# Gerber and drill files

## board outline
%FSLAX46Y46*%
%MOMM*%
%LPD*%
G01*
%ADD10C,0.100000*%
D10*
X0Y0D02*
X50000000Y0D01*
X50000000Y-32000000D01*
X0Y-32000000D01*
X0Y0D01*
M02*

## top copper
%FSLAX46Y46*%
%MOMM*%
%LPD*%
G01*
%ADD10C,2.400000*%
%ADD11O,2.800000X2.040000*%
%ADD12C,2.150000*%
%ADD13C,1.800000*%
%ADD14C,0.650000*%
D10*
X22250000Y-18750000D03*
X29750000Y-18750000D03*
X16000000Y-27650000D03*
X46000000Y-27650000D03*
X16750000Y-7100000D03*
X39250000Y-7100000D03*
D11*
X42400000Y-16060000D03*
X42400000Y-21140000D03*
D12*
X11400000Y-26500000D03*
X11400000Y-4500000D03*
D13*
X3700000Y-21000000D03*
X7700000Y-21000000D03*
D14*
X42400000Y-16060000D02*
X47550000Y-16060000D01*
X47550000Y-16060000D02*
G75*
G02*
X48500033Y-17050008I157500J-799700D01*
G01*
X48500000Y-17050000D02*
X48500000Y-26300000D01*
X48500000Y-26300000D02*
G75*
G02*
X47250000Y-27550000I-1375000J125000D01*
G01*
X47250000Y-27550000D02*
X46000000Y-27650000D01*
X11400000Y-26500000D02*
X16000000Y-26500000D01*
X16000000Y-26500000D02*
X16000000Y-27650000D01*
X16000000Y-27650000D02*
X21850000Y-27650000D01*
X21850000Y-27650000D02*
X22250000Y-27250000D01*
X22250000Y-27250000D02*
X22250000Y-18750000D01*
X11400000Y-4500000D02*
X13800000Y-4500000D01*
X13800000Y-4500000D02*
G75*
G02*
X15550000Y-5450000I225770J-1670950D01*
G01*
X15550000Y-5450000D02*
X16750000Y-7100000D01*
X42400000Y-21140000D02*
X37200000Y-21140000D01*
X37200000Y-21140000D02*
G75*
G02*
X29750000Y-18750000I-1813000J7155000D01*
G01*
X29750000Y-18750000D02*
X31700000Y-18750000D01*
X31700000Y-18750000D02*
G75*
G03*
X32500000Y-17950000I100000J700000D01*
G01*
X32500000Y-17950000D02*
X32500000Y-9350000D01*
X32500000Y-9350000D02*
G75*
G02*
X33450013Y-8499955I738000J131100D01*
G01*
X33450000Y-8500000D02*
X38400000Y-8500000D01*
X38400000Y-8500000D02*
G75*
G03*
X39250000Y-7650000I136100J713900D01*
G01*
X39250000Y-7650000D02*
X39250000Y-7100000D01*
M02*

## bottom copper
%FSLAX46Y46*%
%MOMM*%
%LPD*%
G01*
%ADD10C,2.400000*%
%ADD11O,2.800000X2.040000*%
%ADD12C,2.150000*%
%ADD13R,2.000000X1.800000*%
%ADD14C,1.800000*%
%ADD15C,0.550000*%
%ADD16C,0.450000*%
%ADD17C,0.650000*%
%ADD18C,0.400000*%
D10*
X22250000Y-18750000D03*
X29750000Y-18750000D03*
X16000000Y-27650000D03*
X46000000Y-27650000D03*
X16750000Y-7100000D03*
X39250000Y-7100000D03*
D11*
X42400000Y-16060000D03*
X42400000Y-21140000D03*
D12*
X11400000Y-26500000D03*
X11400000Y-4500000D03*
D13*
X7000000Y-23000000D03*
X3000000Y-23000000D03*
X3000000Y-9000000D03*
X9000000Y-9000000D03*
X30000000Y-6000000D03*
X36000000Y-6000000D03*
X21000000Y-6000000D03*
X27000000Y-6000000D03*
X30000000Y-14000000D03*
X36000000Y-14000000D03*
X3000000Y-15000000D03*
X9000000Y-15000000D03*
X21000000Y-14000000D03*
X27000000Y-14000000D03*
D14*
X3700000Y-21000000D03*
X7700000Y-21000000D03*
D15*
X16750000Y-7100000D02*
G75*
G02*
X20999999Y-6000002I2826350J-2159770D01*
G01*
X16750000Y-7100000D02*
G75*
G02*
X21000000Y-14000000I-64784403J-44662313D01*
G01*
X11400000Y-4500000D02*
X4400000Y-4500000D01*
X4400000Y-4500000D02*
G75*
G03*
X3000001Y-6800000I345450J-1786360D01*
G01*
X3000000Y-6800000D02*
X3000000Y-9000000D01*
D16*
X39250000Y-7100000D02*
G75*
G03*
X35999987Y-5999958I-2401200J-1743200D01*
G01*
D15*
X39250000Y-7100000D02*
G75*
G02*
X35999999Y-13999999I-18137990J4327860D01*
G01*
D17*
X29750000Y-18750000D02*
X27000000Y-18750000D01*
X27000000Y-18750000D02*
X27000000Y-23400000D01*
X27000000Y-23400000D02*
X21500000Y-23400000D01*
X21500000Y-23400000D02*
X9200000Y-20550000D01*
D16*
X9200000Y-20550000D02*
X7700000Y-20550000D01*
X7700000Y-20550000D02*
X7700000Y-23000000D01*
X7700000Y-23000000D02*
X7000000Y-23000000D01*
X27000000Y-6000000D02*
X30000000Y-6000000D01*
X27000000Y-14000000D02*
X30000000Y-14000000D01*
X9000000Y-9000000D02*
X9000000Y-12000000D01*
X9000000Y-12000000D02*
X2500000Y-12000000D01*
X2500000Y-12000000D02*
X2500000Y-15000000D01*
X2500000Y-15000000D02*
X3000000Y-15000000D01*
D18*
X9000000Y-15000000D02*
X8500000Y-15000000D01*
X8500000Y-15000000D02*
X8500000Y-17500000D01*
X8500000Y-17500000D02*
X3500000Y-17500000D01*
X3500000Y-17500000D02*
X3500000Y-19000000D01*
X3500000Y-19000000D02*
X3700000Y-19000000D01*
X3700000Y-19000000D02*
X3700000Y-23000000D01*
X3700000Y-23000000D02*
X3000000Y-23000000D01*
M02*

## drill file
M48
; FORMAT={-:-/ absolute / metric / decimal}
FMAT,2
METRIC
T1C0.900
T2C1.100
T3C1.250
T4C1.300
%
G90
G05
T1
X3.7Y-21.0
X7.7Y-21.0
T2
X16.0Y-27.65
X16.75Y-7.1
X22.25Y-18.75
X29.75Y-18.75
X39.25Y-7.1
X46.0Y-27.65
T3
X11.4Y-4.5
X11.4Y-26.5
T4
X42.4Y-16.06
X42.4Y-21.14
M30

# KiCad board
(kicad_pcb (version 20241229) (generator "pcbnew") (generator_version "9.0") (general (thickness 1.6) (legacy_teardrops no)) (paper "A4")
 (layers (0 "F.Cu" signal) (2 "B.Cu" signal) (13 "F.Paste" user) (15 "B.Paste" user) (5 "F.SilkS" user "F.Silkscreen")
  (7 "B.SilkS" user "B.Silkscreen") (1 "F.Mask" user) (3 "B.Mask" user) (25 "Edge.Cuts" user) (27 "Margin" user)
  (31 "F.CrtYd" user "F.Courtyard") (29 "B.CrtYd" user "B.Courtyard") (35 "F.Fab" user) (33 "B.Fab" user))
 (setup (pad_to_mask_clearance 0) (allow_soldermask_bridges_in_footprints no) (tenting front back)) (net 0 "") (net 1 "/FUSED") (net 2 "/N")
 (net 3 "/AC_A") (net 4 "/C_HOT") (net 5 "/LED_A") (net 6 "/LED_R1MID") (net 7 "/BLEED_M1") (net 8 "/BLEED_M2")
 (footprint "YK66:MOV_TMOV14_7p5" (layer "F.Cu") (at 26 18.75)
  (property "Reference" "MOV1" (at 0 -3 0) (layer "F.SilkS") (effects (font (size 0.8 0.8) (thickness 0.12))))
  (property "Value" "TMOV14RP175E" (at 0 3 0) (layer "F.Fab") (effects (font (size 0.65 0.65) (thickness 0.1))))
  (pad "1" thru_hole circle (at -3.75 0) (size 2.4 2.4) (drill 1.1) (layers "*.Cu" "*.Mask") (remove_unused_layers no) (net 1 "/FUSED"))
  (pad "2" thru_hole circle (at 3.75 0) (size 2.4 2.4) (drill 1.1) (layers "*.Cu" "*.Mask") (remove_unused_layers no) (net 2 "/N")))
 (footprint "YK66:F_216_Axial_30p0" (layer "F.Cu") (at 31 27.65)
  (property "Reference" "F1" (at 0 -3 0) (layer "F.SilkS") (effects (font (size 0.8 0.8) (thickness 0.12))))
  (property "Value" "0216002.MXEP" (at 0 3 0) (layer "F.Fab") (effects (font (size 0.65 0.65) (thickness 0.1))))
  (pad "1" thru_hole circle (at -15 0) (size 2.4 2.4) (drill 1.1) (layers "*.Cu" "*.Mask") (remove_unused_layers no) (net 1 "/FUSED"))
  (pad "2" thru_hole circle (at 15 0) (size 2.4 2.4) (drill 1.1) (layers "*.Cu" "*.Mask") (remove_unused_layers no) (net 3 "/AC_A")))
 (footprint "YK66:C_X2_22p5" (layer "F.Cu") (at 28 7.1)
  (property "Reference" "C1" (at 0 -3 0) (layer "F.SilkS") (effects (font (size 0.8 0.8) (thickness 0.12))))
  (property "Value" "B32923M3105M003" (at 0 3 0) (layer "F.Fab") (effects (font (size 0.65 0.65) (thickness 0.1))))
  (pad "1" thru_hole circle (at -11.25 0) (size 2.4 2.4) (drill 1.1) (layers "*.Cu" "*.Mask") (remove_unused_layers no) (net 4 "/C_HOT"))
  (pad "2" thru_hole circle (at 11.25 0) (size 2.4 2.4) (drill 1.1) (layers "*.Cu" "*.Mask") (remove_unused_layers no) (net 2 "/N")))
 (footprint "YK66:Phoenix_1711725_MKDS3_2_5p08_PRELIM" (layer "F.Cu") (at 42.4 18.6)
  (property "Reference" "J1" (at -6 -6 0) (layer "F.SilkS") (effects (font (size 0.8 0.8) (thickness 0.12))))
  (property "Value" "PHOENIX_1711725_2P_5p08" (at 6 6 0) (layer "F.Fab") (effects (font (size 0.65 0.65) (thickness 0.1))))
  (pad "1" thru_hole oval (at 0 -2.54) (size 2.8 2.04) (drill 1.3) (layers "*.Cu" "*.Mask") (remove_unused_layers no) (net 3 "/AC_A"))
  (pad "2" thru_hole oval (at 0 2.54) (size 2.8 2.04) (drill 1.3) (layers "*.Cu" "*.Mask") (remove_unused_layers no) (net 2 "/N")))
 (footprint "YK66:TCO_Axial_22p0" (layer "F.Cu") (at 11.4 15.5)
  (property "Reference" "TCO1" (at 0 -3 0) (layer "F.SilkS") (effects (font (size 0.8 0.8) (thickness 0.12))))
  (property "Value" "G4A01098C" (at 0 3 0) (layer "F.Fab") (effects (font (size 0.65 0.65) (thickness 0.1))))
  (pad "1" thru_hole circle (at 0 11) (size 2.15 2.15) (drill 1.25) (layers "*.Cu" "*.Mask") (remove_unused_layers no) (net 1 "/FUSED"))
  (pad "2" thru_hole circle (at 0 -11) (size 2.15 2.15) (drill 1.25) (layers "*.Cu" "*.Mask") (remove_unused_layers no) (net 4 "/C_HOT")))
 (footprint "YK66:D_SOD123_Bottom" (layer "B.Cu") (at 5 23)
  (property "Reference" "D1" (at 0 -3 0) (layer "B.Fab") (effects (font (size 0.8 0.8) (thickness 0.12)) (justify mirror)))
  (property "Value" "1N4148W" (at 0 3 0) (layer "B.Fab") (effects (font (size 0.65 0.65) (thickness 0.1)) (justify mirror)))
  (pad "1" smd rect (at 2 0) (size 2 1.8) (layers "B.Cu" "B.Mask" "B.Paste") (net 2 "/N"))
  (pad "2" smd rect (at -2 0) (size 2 1.8) (layers "B.Cu" "B.Mask" "B.Paste") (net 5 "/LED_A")))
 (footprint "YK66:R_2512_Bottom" (layer "B.Cu") (at 6 9)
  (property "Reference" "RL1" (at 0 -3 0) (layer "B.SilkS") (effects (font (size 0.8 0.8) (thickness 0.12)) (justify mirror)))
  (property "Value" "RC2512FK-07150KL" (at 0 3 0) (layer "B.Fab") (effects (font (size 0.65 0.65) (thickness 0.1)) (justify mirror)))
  (pad "1" smd rect (at -3 0) (size 2 1.8) (layers "B.Cu" "B.Mask" "B.Paste") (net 4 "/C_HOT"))
  (pad "2" smd rect (at 3 0) (size 2 1.8) (layers "B.Cu" "B.Mask" "B.Paste") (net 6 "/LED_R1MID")))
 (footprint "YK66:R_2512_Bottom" (layer "B.Cu") (at 33 6)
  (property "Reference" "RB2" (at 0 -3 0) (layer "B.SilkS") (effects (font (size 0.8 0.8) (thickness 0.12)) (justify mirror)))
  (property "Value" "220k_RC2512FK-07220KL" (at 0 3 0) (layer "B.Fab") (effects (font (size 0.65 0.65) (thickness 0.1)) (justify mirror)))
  (pad "1" smd rect (at -3 0) (size 2 1.8) (layers "B.Cu" "B.Mask" "B.Paste") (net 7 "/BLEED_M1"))
  (pad "2" smd rect (at 3 0) (size 2 1.8) (layers "B.Cu" "B.Mask" "B.Paste") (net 2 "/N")))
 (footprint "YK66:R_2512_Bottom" (layer "B.Cu") (at 24 6)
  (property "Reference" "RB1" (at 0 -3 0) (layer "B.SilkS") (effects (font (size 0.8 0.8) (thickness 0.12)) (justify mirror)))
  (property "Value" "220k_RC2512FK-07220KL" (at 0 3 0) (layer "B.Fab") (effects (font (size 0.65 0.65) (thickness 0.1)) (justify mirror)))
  (pad "1" smd rect (at -3 0) (size 2 1.8) (layers "B.Cu" "B.Mask" "B.Paste") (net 4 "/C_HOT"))
  (pad "2" smd rect (at 3 0) (size 2 1.8) (layers "B.Cu" "B.Mask" "B.Paste") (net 7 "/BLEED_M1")))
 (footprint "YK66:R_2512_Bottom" (layer "B.Cu") (at 33 14)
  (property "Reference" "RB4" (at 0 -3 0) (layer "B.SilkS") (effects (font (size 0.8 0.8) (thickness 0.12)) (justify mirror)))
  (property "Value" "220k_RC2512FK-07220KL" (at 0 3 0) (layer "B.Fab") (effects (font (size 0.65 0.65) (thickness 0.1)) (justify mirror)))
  (pad "1" smd rect (at -3 0) (size 2 1.8) (layers "B.Cu" "B.Mask" "B.Paste") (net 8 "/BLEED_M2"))
  (pad "2" smd rect (at 3 0) (size 2 1.8) (layers "B.Cu" "B.Mask" "B.Paste") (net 2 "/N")))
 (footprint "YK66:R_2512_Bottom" (layer "B.Cu") (at 6 15)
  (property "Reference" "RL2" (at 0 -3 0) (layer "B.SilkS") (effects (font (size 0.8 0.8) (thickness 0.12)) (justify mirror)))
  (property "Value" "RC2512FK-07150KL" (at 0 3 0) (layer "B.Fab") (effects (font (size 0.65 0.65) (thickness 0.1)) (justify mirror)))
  (pad "1" smd rect (at -3 0) (size 2 1.8) (layers "B.Cu" "B.Mask" "B.Paste") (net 6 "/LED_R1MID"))
  (pad "2" smd rect (at 3 0) (size 2 1.8) (layers "B.Cu" "B.Mask" "B.Paste") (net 5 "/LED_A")))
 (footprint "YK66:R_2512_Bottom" (layer "B.Cu") (at 24 14)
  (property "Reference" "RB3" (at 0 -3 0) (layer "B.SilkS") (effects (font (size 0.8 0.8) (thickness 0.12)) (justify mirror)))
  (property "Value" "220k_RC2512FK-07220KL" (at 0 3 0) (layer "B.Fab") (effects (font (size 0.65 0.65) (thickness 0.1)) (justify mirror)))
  (pad "1" smd rect (at -3 0) (size 2 1.8) (layers "B.Cu" "B.Mask" "B.Paste") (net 4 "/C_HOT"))
  (pad "2" smd rect (at 3 0) (size 2 1.8) (layers "B.Cu" "B.Mask" "B.Paste") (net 8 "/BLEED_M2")))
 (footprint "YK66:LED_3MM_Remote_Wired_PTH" (layer "F.Cu") (at 5.7 21)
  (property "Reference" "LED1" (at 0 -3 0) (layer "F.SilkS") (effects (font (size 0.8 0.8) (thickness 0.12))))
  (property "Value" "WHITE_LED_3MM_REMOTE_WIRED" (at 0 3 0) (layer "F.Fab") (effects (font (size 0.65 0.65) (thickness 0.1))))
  (pad "1" thru_hole circle (at -2 0) (size 1.8 1.8) (drill 0.9) (layers "*.Cu" "*.Mask") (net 5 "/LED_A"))
  (pad "2" thru_hole circle (at 2 0) (size 1.8 1.8) (drill 0.9) (layers "*.Cu" "*.Mask") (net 2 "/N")))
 (gr_rect (start 0 0) (end 50 32) (stroke (width 0.1) (type default)) (fill no) (layer "Edge.Cuts"))
 (segment (start 42.4000 16.0600) (end 47.5500 16.0600) (width 0.650) (layer "F.Cu") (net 3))
 (arc (start 47.5500 16.0600) (mid 48.3000 16.3000) (end 48.5000 17.0500) (width 0.650) (layer "F.Cu") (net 3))
 (segment (start 48.5000 17.0500) (end 48.5000 26.3000) (width 0.650) (layer "F.Cu") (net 3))
 (arc (start 48.5000 26.3000) (mid 48.1500 27.1000) (end 47.2500 27.5500) (width 0.650) (layer "F.Cu") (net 3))
 (segment (start 47.2500 27.5500) (end 46.0000 27.6500) (width 0.650) (layer "F.Cu") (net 3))
 (segment (start 11.4000 26.5000) (end 16.0000 26.5000) (width 0.650) (layer "F.Cu") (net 1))
 (segment (start 16.0000 26.5000) (end 16.0000 27.6500) (width 0.650) (layer "F.Cu") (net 1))
 (segment (start 16.0000 27.6500) (end 21.8500 27.6500) (width 0.650) (layer "F.Cu") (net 1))
 (segment (start 21.8500 27.6500) (end 22.2500 27.2500) (width 0.650) (layer "F.Cu") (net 1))
 (segment (start 22.2500 27.2500) (end 22.2500 18.7500) (width 0.650) (layer "F.Cu") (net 1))
 (segment (start 11.4000 4.5000) (end 13.8000 4.5000) (width 0.650) (layer "F.Cu") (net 4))
 (arc (start 13.8000 4.5000) (mid 14.8500 4.7000) (end 15.5500 5.4500) (width 0.650) (layer "F.Cu") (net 4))
 (segment (start 15.5500 5.4500) (end 16.7500 7.1000) (width 0.650) (layer "F.Cu") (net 4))
 (arc (start 16.7500 7.1000) (mid 18.7500 5.8000) (end 21.0000 6.0000) (width 0.550) (layer "B.Cu") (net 4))
 (arc (start 16.7500 7.1000) (mid 18.7500 10.1500) (end 21.0000 14.0000) (width 0.550) (layer "B.Cu") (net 4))
 (segment (start 11.4000 4.5000) (end 4.4000 4.5000) (width 0.550) (layer "B.Cu") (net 4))
 (arc (start 4.4000 4.5000) (mid 3.2500 5.2500) (end 3.0000 6.8000) (width 0.550) (layer "B.Cu") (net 4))
 (segment (start 3.0000 6.8000) (end 3.0000 9.0000) (width 0.550) (layer "B.Cu") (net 4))
 (segment (start 42.4000 21.1400) (end 37.2000 21.1400) (width 0.650) (layer "F.Cu") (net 2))
 (arc (start 37.2000 21.1400) (mid 33.2500 21.0500) (end 29.7500 18.7500) (width 0.650) (layer "F.Cu") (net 2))
 (segment (start 29.7500 18.7500) (end 31.7000 18.7500) (width 0.650) (layer "F.Cu") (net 2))
 (arc (start 31.7000 18.7500) (mid 32.3000 18.5500) (end 32.5000 17.9500) (width 0.650) (layer "F.Cu") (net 2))
 (segment (start 32.5000 17.9500) (end 32.5000 9.3500) (width 0.650) (layer "F.Cu") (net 2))
 (arc (start 32.5000 9.3500) (mid 32.7500 8.6500) (end 33.4500 8.5000) (width 0.650) (layer "F.Cu") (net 2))
 (segment (start 33.4500 8.5000) (end 38.4000 8.5000) (width 0.650) (layer "F.Cu") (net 2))
 (arc (start 38.4000 8.5000) (mid 39.0500 8.3000) (end 39.2500 7.6500) (width 0.650) (layer "F.Cu") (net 2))
 (segment (start 39.2500 7.6500) (end 39.2500 7.1000) (width 0.650) (layer "F.Cu") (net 2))
 (arc (start 39.2500 7.1000) (mid 37.8500 6.0500) (end 36.0000 6.0000) (width 0.450) (layer "B.Cu") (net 2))
 (arc (start 39.2500 7.1000) (mid 38.1500 10.3500) (end 36.0000 14.0000) (width 0.550) (layer "B.Cu") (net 2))
 (segment (start 29.7500 18.7500) (end 27.0000 18.7500) (width 0.650) (layer "B.Cu") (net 2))
 (segment (start 27.0000 18.7500) (end 27.0000 23.4000) (width 0.650) (layer "B.Cu") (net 2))
 (segment (start 27.0000 23.4000) (end 21.5000 23.4000) (width 0.650) (layer "B.Cu") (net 2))
 (segment (start 21.5000 23.4000) (end 9.2000 20.5500) (width 0.650) (layer "B.Cu") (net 2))
 (segment (start 9.2000 20.5500) (end 7.7000 20.5500) (width 0.450) (layer "B.Cu") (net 2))
 (segment (start 7.7000 20.5500) (end 7.7000 23.0000) (width 0.450) (layer "B.Cu") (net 2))
 (segment (start 7.7000 23.0000) (end 7.0000 23.0000) (width 0.450) (layer "B.Cu") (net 2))
 (segment (start 27.0000 6.0000) (end 30.0000 6.0000) (width 0.450) (layer "B.Cu") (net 7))
 (segment (start 27.0000 14.0000) (end 30.0000 14.0000) (width 0.450) (layer "B.Cu") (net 8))
 (segment (start 9.0000 9.0000) (end 9.0000 12.0000) (width 0.450) (layer "B.Cu") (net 6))
 (segment (start 9.0000 12.0000) (end 2.5000 12.0000) (width 0.450) (layer "B.Cu") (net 6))
 (segment (start 2.5000 12.0000) (end 2.5000 15.0000) (width 0.450) (layer "B.Cu") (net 6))
 (segment (start 2.5000 15.0000) (end 3.0000 15.0000) (width 0.450) (layer "B.Cu") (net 6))
 (segment (start 9.0000 15.0000) (end 8.5000 15.0000) (width 0.400) (layer "B.Cu") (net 5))
 (segment (start 8.5000 15.0000) (end 8.5000 17.5000) (width 0.400) (layer "B.Cu") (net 5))
 (segment (start 8.5000 17.5000) (end 3.5000 17.5000) (width 0.400) (layer "B.Cu") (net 5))
 (segment (start 3.5000 17.5000) (end 3.5000 19.0000) (width 0.400) (layer "B.Cu") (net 5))
 (segment (start 3.5000 19.0000) (end 3.7000 19.0000) (width 0.400) (layer "B.Cu") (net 5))
 (segment (start 3.7000 19.0000) (end 3.7000 23.0000) (width 0.400) (layer "B.Cu") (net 5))
 (segment (start 3.7000 23.0000) (end 3.0000 23.0000) (width 0.400) (layer "B.Cu") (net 5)))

